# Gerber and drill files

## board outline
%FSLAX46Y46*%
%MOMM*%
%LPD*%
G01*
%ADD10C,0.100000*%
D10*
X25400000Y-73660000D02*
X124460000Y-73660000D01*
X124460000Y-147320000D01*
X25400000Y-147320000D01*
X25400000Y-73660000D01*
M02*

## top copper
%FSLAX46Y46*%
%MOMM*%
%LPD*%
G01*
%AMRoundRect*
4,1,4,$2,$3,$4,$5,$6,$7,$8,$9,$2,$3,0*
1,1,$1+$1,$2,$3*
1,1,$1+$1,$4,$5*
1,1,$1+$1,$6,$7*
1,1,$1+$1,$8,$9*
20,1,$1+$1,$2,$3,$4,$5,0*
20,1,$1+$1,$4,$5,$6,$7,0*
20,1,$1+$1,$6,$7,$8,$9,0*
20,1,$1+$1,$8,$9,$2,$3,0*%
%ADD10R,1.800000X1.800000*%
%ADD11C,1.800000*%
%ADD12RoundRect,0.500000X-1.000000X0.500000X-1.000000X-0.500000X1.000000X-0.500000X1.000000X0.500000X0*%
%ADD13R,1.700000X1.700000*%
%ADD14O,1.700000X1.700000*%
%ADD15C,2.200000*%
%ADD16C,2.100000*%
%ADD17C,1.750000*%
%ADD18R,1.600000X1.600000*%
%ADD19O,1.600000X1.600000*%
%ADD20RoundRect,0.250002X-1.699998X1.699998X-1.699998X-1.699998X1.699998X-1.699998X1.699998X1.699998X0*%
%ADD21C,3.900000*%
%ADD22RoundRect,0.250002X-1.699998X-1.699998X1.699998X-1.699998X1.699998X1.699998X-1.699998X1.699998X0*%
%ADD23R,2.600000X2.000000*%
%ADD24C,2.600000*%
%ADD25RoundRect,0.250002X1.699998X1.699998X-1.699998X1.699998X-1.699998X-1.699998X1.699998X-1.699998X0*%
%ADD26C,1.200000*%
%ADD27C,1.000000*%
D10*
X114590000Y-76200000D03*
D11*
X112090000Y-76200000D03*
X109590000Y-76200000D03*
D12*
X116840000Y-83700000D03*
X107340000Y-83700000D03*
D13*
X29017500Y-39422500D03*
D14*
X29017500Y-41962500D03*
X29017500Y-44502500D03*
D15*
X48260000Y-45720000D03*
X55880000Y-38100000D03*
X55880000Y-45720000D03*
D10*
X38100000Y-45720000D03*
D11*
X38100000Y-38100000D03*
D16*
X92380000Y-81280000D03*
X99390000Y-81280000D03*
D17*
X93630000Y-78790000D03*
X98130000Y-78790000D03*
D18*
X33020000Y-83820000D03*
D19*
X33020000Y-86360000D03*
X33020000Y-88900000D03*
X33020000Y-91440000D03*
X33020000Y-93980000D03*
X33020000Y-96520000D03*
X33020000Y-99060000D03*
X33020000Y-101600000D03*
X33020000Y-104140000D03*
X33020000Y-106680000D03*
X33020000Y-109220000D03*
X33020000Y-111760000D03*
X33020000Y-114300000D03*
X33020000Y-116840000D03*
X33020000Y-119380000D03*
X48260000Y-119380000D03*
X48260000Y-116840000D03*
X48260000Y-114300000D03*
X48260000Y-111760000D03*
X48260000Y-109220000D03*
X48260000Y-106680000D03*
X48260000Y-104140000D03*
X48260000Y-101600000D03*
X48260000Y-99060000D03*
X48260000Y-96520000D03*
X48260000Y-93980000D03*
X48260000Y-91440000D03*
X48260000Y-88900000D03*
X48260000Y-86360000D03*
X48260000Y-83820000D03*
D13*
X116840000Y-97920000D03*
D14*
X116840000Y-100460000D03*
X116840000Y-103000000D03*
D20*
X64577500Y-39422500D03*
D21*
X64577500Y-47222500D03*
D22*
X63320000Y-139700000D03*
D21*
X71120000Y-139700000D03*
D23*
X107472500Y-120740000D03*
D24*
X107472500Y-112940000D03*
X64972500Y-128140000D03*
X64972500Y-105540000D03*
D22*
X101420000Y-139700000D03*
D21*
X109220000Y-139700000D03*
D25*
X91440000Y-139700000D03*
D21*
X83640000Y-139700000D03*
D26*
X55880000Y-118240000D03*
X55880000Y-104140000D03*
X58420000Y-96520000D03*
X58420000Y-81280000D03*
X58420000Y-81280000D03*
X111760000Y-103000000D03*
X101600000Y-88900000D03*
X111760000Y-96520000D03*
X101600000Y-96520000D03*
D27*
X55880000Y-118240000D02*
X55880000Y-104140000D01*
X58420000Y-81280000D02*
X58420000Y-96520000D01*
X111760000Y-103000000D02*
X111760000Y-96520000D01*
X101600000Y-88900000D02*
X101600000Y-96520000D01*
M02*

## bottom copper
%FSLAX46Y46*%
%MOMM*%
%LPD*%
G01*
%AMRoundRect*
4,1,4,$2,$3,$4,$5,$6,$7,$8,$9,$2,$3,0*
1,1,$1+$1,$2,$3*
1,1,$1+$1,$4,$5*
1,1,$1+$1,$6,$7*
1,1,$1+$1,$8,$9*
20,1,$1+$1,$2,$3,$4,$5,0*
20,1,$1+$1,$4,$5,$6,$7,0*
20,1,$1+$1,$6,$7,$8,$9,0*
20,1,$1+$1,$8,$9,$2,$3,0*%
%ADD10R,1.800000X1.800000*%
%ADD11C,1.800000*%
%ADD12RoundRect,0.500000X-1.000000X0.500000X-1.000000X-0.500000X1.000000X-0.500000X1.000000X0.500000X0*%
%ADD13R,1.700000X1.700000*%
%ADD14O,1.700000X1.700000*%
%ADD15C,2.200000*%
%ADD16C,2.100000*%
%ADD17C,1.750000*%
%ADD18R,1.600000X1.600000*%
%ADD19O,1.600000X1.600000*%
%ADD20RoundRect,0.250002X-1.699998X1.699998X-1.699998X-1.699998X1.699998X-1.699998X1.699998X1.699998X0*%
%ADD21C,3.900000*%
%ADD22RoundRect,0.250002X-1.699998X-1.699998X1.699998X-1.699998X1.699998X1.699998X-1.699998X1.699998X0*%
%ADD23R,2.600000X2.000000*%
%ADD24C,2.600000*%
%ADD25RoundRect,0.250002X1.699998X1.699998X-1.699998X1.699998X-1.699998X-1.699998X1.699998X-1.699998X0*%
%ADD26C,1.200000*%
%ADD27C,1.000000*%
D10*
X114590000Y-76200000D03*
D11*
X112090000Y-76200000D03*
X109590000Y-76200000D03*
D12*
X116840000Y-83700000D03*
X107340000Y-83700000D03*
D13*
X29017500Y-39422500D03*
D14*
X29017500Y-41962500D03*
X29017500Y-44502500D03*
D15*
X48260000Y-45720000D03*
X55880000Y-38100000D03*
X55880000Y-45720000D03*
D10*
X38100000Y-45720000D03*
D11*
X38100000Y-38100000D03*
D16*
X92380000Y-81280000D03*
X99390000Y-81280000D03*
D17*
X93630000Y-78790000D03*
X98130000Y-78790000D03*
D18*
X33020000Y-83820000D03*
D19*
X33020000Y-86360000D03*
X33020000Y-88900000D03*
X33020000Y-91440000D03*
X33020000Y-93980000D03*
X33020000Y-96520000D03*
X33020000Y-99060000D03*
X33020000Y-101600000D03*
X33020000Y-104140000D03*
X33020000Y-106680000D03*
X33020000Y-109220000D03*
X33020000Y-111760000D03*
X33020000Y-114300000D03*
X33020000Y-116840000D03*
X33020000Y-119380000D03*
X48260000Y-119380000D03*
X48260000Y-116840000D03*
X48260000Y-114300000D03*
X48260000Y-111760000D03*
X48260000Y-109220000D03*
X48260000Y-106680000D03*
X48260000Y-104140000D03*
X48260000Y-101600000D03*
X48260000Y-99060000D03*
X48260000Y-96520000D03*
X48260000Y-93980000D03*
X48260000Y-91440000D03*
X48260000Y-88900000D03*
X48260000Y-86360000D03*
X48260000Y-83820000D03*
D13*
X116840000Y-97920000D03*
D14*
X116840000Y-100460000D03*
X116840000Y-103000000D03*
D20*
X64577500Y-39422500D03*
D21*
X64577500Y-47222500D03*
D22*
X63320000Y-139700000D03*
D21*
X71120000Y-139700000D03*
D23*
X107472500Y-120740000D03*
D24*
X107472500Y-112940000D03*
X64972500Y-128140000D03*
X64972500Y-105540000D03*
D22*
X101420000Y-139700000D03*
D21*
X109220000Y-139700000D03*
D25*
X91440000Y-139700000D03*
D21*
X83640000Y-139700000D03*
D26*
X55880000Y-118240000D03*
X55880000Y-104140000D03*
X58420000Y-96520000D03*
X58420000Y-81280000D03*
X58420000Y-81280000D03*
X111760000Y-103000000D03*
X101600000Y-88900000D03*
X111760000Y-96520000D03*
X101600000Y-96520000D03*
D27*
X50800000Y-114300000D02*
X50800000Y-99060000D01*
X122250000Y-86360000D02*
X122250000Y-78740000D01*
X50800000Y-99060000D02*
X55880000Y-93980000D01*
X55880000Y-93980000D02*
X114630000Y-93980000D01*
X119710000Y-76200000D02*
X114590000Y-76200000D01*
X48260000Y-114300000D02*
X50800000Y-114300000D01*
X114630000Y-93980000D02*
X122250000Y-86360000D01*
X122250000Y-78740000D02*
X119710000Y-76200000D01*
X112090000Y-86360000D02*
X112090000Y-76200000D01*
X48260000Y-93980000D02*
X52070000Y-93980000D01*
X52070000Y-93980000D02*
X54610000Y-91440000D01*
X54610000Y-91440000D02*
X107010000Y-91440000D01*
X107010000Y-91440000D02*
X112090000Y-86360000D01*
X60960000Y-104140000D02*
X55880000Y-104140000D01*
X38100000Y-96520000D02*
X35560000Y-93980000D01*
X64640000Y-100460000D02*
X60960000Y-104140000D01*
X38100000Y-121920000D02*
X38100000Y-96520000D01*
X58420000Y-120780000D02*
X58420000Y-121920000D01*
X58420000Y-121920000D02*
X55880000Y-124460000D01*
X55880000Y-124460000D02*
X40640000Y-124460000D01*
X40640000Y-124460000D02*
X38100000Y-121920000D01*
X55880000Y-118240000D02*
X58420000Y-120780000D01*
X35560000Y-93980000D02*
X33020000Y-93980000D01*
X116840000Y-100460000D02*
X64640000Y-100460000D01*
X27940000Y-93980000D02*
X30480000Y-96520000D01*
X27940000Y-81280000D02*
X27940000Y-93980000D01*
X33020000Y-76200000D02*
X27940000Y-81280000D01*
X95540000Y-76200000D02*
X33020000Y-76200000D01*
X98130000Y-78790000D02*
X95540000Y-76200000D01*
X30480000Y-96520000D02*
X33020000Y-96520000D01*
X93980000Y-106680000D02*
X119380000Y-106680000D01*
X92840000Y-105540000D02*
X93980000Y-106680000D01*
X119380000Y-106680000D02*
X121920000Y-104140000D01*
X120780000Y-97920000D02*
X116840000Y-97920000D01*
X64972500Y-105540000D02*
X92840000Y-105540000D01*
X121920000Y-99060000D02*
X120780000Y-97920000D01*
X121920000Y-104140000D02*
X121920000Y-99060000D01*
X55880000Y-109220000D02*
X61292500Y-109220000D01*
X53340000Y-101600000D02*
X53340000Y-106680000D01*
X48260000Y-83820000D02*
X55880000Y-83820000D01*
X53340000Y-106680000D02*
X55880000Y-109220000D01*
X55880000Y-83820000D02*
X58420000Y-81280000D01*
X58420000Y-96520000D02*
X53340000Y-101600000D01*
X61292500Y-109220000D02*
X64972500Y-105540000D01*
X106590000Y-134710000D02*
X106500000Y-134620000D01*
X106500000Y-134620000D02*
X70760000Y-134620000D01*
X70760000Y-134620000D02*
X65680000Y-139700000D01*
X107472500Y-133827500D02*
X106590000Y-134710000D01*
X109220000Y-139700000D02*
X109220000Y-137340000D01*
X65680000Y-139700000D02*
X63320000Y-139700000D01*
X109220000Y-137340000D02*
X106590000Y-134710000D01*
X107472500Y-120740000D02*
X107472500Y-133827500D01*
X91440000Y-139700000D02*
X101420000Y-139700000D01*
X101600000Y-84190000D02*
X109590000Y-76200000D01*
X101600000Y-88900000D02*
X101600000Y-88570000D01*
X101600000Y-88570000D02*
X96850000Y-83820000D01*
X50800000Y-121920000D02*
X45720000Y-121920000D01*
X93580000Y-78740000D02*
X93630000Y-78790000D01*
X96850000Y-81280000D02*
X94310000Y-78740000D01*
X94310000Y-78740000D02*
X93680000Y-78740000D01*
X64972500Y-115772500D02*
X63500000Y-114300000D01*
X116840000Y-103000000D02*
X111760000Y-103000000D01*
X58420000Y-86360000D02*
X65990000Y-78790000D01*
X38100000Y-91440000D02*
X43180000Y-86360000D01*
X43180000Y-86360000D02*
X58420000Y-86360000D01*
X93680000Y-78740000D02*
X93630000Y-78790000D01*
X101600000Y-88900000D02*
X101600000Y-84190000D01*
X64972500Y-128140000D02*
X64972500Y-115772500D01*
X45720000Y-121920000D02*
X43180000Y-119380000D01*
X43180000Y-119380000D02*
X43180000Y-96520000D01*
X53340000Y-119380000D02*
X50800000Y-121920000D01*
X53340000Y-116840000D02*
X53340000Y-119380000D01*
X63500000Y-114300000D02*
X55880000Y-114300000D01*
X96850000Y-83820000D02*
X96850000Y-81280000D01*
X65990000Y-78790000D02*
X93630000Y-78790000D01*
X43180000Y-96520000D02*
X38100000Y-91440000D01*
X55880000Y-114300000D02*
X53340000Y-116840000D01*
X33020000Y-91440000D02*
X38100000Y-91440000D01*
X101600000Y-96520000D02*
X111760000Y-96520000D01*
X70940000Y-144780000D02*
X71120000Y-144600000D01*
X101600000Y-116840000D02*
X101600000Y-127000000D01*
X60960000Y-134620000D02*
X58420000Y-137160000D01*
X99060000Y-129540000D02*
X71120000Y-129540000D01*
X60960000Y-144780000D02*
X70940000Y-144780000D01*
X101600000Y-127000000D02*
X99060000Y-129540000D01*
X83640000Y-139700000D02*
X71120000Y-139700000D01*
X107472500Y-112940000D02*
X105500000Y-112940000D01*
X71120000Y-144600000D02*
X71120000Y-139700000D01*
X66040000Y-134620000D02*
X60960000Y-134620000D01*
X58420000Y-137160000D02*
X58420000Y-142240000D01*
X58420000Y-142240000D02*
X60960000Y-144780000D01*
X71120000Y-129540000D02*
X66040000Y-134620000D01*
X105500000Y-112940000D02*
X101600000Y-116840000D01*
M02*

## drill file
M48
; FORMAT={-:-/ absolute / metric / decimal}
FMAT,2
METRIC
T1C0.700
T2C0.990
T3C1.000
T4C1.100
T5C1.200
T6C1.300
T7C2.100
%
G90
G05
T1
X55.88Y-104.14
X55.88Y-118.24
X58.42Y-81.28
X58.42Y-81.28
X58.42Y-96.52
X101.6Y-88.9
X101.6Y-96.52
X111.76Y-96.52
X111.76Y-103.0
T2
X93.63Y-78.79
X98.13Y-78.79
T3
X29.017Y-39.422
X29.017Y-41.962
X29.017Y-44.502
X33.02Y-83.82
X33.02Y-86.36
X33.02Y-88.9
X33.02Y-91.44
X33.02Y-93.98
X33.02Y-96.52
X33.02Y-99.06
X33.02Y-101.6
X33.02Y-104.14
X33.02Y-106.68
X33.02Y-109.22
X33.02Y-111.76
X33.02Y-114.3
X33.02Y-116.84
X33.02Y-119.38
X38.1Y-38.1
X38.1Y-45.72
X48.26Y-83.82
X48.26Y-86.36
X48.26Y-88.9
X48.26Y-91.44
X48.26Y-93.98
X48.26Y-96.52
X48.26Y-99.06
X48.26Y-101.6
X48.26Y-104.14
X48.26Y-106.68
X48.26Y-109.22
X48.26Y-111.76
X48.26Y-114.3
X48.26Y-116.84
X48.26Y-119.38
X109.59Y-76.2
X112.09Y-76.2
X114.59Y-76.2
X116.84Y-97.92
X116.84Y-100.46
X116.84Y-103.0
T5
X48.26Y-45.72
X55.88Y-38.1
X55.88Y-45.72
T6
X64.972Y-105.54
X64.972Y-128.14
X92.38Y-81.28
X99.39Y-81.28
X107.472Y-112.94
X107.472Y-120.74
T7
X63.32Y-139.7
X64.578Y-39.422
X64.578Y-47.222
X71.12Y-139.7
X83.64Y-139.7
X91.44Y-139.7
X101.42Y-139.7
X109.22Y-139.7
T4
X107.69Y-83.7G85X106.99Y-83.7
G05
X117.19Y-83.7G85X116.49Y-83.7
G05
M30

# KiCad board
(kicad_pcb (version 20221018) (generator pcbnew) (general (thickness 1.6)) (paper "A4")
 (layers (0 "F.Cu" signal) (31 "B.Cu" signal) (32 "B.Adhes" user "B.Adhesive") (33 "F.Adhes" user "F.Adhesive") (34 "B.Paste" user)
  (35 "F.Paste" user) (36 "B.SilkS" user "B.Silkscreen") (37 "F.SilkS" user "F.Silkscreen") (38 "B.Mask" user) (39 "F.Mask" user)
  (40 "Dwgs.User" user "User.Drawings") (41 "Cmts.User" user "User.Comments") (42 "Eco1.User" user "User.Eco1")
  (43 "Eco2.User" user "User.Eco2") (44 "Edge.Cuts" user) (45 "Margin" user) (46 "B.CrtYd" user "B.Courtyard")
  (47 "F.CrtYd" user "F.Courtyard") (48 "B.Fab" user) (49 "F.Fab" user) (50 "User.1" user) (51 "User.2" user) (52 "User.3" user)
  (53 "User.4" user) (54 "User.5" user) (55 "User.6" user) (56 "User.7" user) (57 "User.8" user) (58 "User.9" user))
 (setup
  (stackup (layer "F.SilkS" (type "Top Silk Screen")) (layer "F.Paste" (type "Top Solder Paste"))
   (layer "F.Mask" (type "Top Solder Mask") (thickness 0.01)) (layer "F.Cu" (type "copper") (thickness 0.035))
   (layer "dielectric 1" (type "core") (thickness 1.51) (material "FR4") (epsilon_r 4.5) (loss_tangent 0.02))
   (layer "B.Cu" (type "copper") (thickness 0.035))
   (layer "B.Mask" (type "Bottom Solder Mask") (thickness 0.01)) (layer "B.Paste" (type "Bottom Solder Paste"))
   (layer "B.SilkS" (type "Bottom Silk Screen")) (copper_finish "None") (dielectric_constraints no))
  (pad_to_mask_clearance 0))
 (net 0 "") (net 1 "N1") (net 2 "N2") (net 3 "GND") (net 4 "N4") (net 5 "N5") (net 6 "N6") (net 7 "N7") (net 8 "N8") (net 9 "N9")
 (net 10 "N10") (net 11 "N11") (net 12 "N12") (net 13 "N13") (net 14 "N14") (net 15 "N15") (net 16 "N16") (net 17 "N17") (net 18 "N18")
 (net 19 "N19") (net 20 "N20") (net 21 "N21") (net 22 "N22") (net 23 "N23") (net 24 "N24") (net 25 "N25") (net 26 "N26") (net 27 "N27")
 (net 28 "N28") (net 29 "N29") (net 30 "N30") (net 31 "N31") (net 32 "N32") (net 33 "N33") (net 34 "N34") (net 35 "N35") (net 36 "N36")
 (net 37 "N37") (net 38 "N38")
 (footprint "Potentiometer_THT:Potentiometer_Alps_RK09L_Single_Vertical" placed (layer "F.Cu") (at 114.59 76.2 -90)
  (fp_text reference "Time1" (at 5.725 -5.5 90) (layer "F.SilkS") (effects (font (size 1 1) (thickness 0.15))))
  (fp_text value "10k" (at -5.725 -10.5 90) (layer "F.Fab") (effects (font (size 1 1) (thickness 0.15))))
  (pad "1" thru_hole rect (at 0 0 270) (size 1.8 1.8) (drill 1) (layers "*.Cu" "*.Mask") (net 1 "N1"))
  (pad "2" thru_hole circle (at 0 2.5 270) (size 1.8 1.8) (drill 1) (layers "*.Cu" "*.Mask") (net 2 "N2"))
  (pad "3" thru_hole circle (at 0 5 270) (size 1.8 1.8) (drill 1) (layers "*.Cu" "*.Mask") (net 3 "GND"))
  (pad "MP" thru_hole roundrect (at 7.5 -2.25 270) (size 2 3) (drill oval 1.1 1.8) (layers "*.Cu" "*.Mask") (roundrect_rratio 0.25))
  (pad "MP" thru_hole roundrect (at 7.5 7.25 270) (size 2 3) (drill oval 1.1 1.8) (layers "*.Cu" "*.Mask") (roundrect_rratio 0.25))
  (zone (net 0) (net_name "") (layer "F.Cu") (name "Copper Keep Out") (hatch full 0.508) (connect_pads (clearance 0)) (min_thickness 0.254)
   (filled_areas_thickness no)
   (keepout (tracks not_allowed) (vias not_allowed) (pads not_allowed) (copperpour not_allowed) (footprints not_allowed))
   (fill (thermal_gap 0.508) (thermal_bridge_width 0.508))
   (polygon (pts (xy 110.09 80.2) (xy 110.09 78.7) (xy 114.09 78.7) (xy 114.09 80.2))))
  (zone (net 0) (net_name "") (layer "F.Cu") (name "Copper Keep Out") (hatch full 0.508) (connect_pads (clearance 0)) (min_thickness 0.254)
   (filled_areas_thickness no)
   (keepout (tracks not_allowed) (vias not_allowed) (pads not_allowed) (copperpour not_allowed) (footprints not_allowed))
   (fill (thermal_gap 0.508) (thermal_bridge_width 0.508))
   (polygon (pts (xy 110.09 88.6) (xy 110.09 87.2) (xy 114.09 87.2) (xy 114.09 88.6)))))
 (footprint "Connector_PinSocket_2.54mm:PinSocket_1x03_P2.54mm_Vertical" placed (layer "F.Cu") (at 29.0175 39.4225)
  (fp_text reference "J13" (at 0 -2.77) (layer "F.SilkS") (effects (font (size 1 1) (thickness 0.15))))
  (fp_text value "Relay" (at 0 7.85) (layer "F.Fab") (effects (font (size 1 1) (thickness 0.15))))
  (pad "1" thru_hole rect (at 0 0) (size 1.7 1.7) (drill 1) (layers "*.Cu" "*.Mask") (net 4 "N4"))
  (pad "2" thru_hole oval (at 0 2.54) (size 1.7 1.7) (drill 1) (layers "*.Cu" "*.Mask") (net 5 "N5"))
  (pad "3" thru_hole oval (at 0 5.08) (size 1.7 1.7) (drill 1) (layers "*.Cu" "*.Mask") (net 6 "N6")))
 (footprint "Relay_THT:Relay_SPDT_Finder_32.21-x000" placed (layer "F.Cu") (at 38.1 45.72)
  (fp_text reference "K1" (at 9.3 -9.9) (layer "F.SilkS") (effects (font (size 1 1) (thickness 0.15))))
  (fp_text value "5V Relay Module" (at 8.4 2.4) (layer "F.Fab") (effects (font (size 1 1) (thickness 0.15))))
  (pad "11" thru_hole circle (at 10.16 0 90) (size 2.2 2.2) (drill 1.2) (layers "*.Cu" "*.Mask") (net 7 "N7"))
  (pad "12" thru_hole circle (at 17.78 -7.62 90) (size 2.2 2.2) (drill 1.2) (layers "*.Cu" "*.Mask") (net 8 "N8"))
  (pad "14" thru_hole circle (at 17.78 0 90) (size 2.2 2.2) (drill 1.2) (layers "*.Cu" "*.Mask") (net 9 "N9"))
  (pad "A1" thru_hole rect (at 0 0 90) (size 1.8 1.8) (drill 1) (layers "*.Cu" "*.Mask") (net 6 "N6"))
  (pad "A2" thru_hole circle (at 0 -7.62 90) (size 1.8 1.8) (drill 1) (layers "*.Cu" "*.Mask") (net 5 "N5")))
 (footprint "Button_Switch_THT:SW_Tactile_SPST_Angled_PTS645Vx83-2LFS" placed (layer "F.Cu") (at 93.63 78.79)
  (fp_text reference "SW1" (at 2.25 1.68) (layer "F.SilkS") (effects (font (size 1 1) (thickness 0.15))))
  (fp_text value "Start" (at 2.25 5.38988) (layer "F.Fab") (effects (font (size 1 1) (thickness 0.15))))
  (pad "" thru_hole circle (at -1.25 2.49) (size 2.1 2.1) (drill 1.3) (layers "*.Cu" "*.Mask"))
  (pad "" thru_hole circle (at 5.76 2.49) (size 2.1 2.1) (drill 1.3) (layers "*.Cu" "*.Mask"))
  (pad "1" thru_hole circle (at 0 0) (size 1.75 1.75) (drill 0.99) (layers "*.Cu" "*.Mask") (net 3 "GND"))
  (pad "2" thru_hole circle (at 4.5 0) (size 1.75 1.75) (drill 0.99) (layers "*.Cu" "*.Mask") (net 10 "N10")))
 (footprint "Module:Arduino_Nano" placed (layer "F.Cu") (at 33.02 83.82)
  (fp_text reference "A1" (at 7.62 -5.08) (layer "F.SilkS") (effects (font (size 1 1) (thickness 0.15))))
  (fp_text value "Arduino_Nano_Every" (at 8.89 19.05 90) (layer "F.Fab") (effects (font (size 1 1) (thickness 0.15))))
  (pad "1" thru_hole rect (at 0 0) (size 1.6 1.6) (drill 1) (layers "*.Cu" "*.Mask") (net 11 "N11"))
  (pad "2" thru_hole oval (at 0 2.54) (size 1.6 1.6) (drill 1) (layers "*.Cu" "*.Mask") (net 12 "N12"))
  (pad "3" thru_hole oval (at 0 5.08) (size 1.6 1.6) (drill 1) (layers "*.Cu" "*.Mask") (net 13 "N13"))
  (pad "4" thru_hole oval (at 0 7.62) (size 1.6 1.6) (drill 1) (layers "*.Cu" "*.Mask") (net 3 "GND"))
  (pad "5" thru_hole oval (at 0 10.16) (size 1.6 1.6) (drill 1) (layers "*.Cu" "*.Mask") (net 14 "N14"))
  (pad "6" thru_hole oval (at 0 12.7) (size 1.6 1.6) (drill 1) (layers "*.Cu" "*.Mask") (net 10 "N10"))
  (pad "7" thru_hole oval (at 0 15.24) (size 1.6 1.6) (drill 1) (layers "*.Cu" "*.Mask") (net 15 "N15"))
  (pad "8" thru_hole oval (at 0 17.78) (size 1.6 1.6) (drill 1) (layers "*.Cu" "*.Mask") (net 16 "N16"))
  (pad "9" thru_hole oval (at 0 20.32) (size 1.6 1.6) (drill 1) (layers "*.Cu" "*.Mask") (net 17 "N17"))
  (pad "10" thru_hole oval (at 0 22.86) (size 1.6 1.6) (drill 1) (layers "*.Cu" "*.Mask") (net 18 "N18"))
  (pad "11" thru_hole oval (at 0 25.4) (size 1.6 1.6) (drill 1) (layers "*.Cu" "*.Mask") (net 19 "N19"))
  (pad "12" thru_hole oval (at 0 27.94) (size 1.6 1.6) (drill 1) (layers "*.Cu" "*.Mask") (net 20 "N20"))
  (pad "13" thru_hole oval (at 0 30.48) (size 1.6 1.6) (drill 1) (layers "*.Cu" "*.Mask") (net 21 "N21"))
  (pad "14" thru_hole oval (at 0 33.02) (size 1.6 1.6) (drill 1) (layers "*.Cu" "*.Mask") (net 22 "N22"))
  (pad "15" thru_hole oval (at 0 35.56) (size 1.6 1.6) (drill 1) (layers "*.Cu" "*.Mask") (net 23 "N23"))
  (pad "16" thru_hole oval (at 15.24 35.56) (size 1.6 1.6) (drill 1) (layers "*.Cu" "*.Mask") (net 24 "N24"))
  (pad "17" thru_hole oval (at 15.24 33.02) (size 1.6 1.6) (drill 1) (layers "*.Cu" "*.Mask") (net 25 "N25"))
  (pad "18" thru_hole oval (at 15.24 30.48) (size 1.6 1.6) (drill 1) (layers "*.Cu" "*.Mask") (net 1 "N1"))
  (pad "19" thru_hole oval (at 15.24 27.94) (size 1.6 1.6) (drill 1) (layers "*.Cu" "*.Mask") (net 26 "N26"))
  (pad "20" thru_hole oval (at 15.24 25.4) (size 1.6 1.6) (drill 1) (layers "*.Cu" "*.Mask") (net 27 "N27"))
  (pad "21" thru_hole oval (at 15.24 22.86) (size 1.6 1.6) (drill 1) (layers "*.Cu" "*.Mask") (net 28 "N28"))
  (pad "22" thru_hole oval (at 15.24 20.32) (size 1.6 1.6) (drill 1) (layers "*.Cu" "*.Mask") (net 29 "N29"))
  (pad "23" thru_hole oval (at 15.24 17.78) (size 1.6 1.6) (drill 1) (layers "*.Cu" "*.Mask") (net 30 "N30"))
  (pad "24" thru_hole oval (at 15.24 15.24) (size 1.6 1.6) (drill 1) (layers "*.Cu" "*.Mask") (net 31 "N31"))
  (pad "25" thru_hole oval (at 15.24 12.7) (size 1.6 1.6) (drill 1) (layers "*.Cu" "*.Mask") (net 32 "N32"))
  (pad "26" thru_hole oval (at 15.24 10.16) (size 1.6 1.6) (drill 1) (layers "*.Cu" "*.Mask") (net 2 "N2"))
  (pad "27" thru_hole oval (at 15.24 7.62) (size 1.6 1.6) (drill 1) (layers "*.Cu" "*.Mask") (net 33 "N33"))
  (pad "28" thru_hole oval (at 15.24 5.08) (size 1.6 1.6) (drill 1) (layers "*.Cu" "*.Mask") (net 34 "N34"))
  (pad "29" thru_hole oval (at 15.24 2.54) (size 1.6 1.6) (drill 1) (layers "*.Cu" "*.Mask") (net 3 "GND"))
  (pad "30" thru_hole oval (at 15.24 0) (size 1.6 1.6) (drill 1) (layers "*.Cu" "*.Mask") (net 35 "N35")))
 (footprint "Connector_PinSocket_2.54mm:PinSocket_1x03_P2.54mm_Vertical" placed (layer "F.Cu") (at 116.84 97.92)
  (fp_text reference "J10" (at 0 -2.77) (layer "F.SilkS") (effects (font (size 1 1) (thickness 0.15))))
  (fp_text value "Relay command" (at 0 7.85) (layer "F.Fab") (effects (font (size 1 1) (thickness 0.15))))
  (pad "1" thru_hole rect (at 0 0) (size 1.7 1.7) (drill 1) (layers "*.Cu" "*.Mask") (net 35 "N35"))
  (pad "2" thru_hole oval (at 0 2.54) (size 1.7 1.7) (drill 1) (layers "*.Cu" "*.Mask") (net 14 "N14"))
  (pad "3" thru_hole oval (at 0 5.08) (size 1.7 1.7) (drill 1) (layers "*.Cu" "*.Mask") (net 3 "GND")))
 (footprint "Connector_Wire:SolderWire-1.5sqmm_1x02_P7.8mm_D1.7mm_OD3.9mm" (layer "F.Cu") (at 64.5775 39.4225 -90)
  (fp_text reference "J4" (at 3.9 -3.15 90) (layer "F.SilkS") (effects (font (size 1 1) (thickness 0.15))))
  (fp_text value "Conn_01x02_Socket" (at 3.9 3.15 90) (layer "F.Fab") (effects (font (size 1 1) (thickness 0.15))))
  (pad "1" thru_hole roundrect (at 0 0 270) (size 3.9 3.9) (drill 2.1) (layers "*.Cu" "*.Mask") (roundrect_rratio 0.064103) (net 7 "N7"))
  (pad "2" thru_hole circle (at 7.8 0 270) (size 3.9 3.9) (drill 2.1) (layers "*.Cu" "*.Mask") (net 9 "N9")))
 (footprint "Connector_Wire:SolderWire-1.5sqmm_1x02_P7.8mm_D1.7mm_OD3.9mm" (layer "F.Cu") (at 63.32 139.7)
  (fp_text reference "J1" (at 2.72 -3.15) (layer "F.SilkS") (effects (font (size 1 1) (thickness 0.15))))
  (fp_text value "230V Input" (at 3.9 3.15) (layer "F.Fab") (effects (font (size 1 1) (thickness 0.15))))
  (pad "1" thru_hole roundrect (at 0 0) (size 3.9 3.9) (drill 2.1) (layers "*.Cu" "*.Mask") (roundrect_rratio 0.064103) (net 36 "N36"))
  (pad "2" thru_hole circle (at 7.8 0) (size 3.9 3.9) (drill 2.1) (layers "*.Cu" "*.Mask") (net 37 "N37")))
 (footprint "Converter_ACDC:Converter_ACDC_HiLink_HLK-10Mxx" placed (layer "F.Cu") (at 107.4725 120.74 180)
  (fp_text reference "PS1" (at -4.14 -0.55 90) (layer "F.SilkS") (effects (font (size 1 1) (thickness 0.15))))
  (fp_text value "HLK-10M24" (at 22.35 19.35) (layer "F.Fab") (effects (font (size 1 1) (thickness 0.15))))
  (pad "1" thru_hole rect (at 0 0 180) (size 2.6 2) (drill 1.3) (layers "*.Cu" "*.Mask") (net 36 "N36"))
  (pad "2" thru_hole circle (at 0 7.8 180) (size 2.6 2.6) (drill 1.3) (layers "*.Cu" "*.Mask") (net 37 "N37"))
  (pad "3" thru_hole circle (at 42.5 -7.4 180) (size 2.6 2.6) (drill 1.3) (layers "*.Cu" "*.Mask") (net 3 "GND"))
  (pad "4" thru_hole circle (at 42.5 15.2 180) (size 2.6 2.6) (drill 1.3) (layers "*.Cu" "*.Mask") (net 35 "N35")))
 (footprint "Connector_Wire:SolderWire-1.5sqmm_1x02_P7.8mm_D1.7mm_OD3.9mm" (layer "F.Cu") (at 101.42 139.7)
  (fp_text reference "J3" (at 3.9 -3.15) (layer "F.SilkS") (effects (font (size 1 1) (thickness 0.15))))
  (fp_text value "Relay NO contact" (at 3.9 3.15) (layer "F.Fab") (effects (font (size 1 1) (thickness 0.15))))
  (pad "1" thru_hole roundrect (at 0 0) (size 3.9 3.9) (drill 2.1) (layers "*.Cu" "*.Mask") (roundrect_rratio 0.064103) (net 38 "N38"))
  (pad "2" thru_hole circle (at 7.8 0) (size 3.9 3.9) (drill 2.1) (layers "*.Cu" "*.Mask") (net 36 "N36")))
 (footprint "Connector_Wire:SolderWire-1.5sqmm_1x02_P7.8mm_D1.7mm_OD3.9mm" (layer "F.Cu") (at 91.44 139.7 180)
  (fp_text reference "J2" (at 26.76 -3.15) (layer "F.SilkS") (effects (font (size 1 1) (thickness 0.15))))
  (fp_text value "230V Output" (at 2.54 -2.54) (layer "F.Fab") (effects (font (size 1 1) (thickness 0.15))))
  (pad "1" thru_hole roundrect (at 0 0 180) (size 3.9 3.9) (drill 2.1) (layers "*.Cu" "*.Mask") (roundrect_rratio 0.064103) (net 38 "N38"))
  (pad "2" thru_hole circle (at 7.8 0 180) (size 3.9 3.9) (drill 2.1) (layers "*.Cu" "*.Mask") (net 37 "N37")))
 (gr_rect (start 25.4 73.66) (end 124.46 147.32) (stroke (width 0.1) (type default)) (fill none) (layer "Edge.Cuts"))
 (segment (start 50.8 114.3) (end 50.8 99.06) (width 1) (layer "B.Cu") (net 1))
 (segment (start 122.25 86.36) (end 122.25 78.74) (width 1) (layer "B.Cu") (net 1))
 (segment (start 50.8 99.06) (end 55.88 93.98) (width 1) (layer "B.Cu") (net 1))
 (segment (start 55.88 93.98) (end 114.63 93.98) (width 1) (layer "B.Cu") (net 1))
 (segment (start 119.71 76.2) (end 114.59 76.2) (width 1) (layer "B.Cu") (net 1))
 (segment (start 48.26 114.3) (end 50.8 114.3) (width 1) (layer "B.Cu") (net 1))
 (segment (start 114.63 93.98) (end 122.25 86.36) (width 1) (layer "B.Cu") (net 1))
 (segment (start 122.25 78.74) (end 119.71 76.2) (width 1) (layer "B.Cu") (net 1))
 (segment (start 112.09 86.36) (end 112.09 76.2) (width 1) (layer "B.Cu") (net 2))
 (segment (start 48.26 93.98) (end 52.07 93.98) (width 1) (layer "B.Cu") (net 2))
 (segment (start 52.07 93.98) (end 54.61 91.44) (width 1) (layer "B.Cu") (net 2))
 (segment (start 54.61 91.44) (end 107.01 91.44) (width 1) (layer "B.Cu") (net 2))
 (segment (start 107.01 91.44) (end 112.09 86.36) (width 1) (layer "B.Cu") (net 2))
 (segment (start 55.88 118.24) (end 55.88 104.14) (width 1) (layer "F.Cu") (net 14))
 (via (at 55.88 118.24) (size 1.2) (drill 0.7) (layers "F.Cu" "B.Cu") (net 14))
 (via (at 55.88 104.14) (size 1.2) (drill 0.7) (layers "F.Cu" "B.Cu") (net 14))
 (segment (start 60.96 104.14) (end 55.88 104.14) (width 1) (layer "B.Cu") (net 14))
 (segment (start 38.1 96.52) (end 35.56 93.98) (width 1) (layer "B.Cu") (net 14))
 (segment (start 64.64 100.46) (end 60.96 104.14) (width 1) (layer "B.Cu") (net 14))
 (segment (start 38.1 121.92) (end 38.1 96.52) (width 1) (layer "B.Cu") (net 14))
 (segment (start 58.42 120.78) (end 58.42 121.92) (width 1) (layer "B.Cu") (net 14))
 (segment (start 58.42 121.92) (end 55.88 124.46) (width 1) (layer "B.Cu") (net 14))
 (segment (start 55.88 124.46) (end 40.64 124.46) (width 1) (layer "B.Cu") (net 14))
 (segment (start 40.64 124.46) (end 38.1 121.92) (width 1) (layer "B.Cu") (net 14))
 (segment (start 55.88 118.24) (end 58.42 120.78) (width 1) (layer "B.Cu") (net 14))
 (segment (start 35.56 93.98) (end 33.02 93.98) (width 1) (layer "B.Cu") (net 14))
 (segment (start 116.84 100.46) (end 64.64 100.46) (width 1) (layer "B.Cu") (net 14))
 (segment (start 27.94 93.98) (end 30.48 96.52) (width 1) (layer "B.Cu") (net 10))
 (segment (start 27.94 81.28) (end 27.94 93.98) (width 1) (layer "B.Cu") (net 10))
 (segment (start 33.02 76.2) (end 27.94 81.28) (width 1) (layer "B.Cu") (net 10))
 (segment (start 95.54 76.2) (end 33.02 76.2) (width 1) (layer "B.Cu") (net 10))
 (segment (start 98.13 78.79) (end 95.54 76.2) (width 1) (layer "B.Cu") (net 10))
 (segment (start 30.48 96.52) (end 33.02 96.52) (width 1) (layer "B.Cu") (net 10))
 (segment (start 58.42 81.28) (end 58.42 96.52) (width 1) (layer "F.Cu") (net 35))
 (via (at 58.42 96.52) (size 1.2) (drill 0.7) (layers "F.Cu" "B.Cu") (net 35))
 (via (at 58.42 81.28) (size 1.2) (drill 0.7) (layers "F.Cu" "B.Cu") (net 35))
 (via (at 58.42 81.28) (size 1.2) (drill 0.7) (layers "F.Cu" "B.Cu") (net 35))
 (segment (start 93.98 106.68) (end 119.38 106.68) (width 1) (layer "B.Cu") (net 35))
 (segment (start 92.84 105.54) (end 93.98 106.68) (width 1) (layer "B.Cu") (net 35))
 (segment (start 119.38 106.68) (end 121.92 104.14) (width 1) (layer "B.Cu") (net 35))
 (segment (start 120.78 97.92) (end 116.84 97.92) (width 1) (layer "B.Cu") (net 35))
 (segment (start 64.9725 105.54) (end 92.84 105.54) (width 1) (layer "B.Cu") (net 35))
 (segment (start 121.92 99.06) (end 120.78 97.92) (width 1) (layer "B.Cu") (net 35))
 (segment (start 121.92 104.14) (end 121.92 99.06) (width 1) (layer "B.Cu") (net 35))
 (segment (start 55.88 109.22) (end 61.2925 109.22) (width 1) (layer "B.Cu") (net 35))
 (segment (start 53.34 101.6) (end 53.34 106.68) (width 1) (layer "B.Cu") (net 35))
 (segment (start 48.26 83.82) (end 55.88 83.82) (width 1) (layer "B.Cu") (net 35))
 (segment (start 53.34 106.68) (end 55.88 109.22) (width 1) (layer "B.Cu") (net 35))
 (segment (start 55.88 83.82) (end 58.42 81.28) (width 1) (layer "B.Cu") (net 35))
 (segment (start 58.42 96.52) (end 53.34 101.6) (width 1) (layer "B.Cu") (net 35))
 (segment (start 61.2925 109.22) (end 64.9725 105.54) (width 1) (layer "B.Cu") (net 35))
 (segment (start 106.59 134.71) (end 106.5 134.62) (width 1) (layer "B.Cu") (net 36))
 (segment (start 106.5 134.62) (end 70.76 134.62) (width 1) (layer "B.Cu") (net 36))
 (segment (start 70.76 134.62) (end 65.68 139.7) (width 1) (layer "B.Cu") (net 36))
 (segment (start 107.4725 133.8275) (end 106.59 134.71) (width 1) (layer "B.Cu") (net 36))
 (segment (start 109.22 139.7) (end 109.22 137.34) (width 1) (layer "B.Cu") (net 36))
 (segment (start 65.68 139.7) (end 63.32 139.7) (width 1) (layer "B.Cu") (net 36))
 (segment (start 109.22 137.34) (end 106.59 134.71) (width 1) (layer "B.Cu") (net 36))
 (segment (start 107.4725 120.74) (end 107.4725 133.8275) (width 1) (layer "B.Cu") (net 36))
 (segment (start 91.44 139.7) (end 101.42 139.7) (width 1) (layer "B.Cu") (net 38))
 (segment (start 111.76 103) (end 111.76 96.52) (width 1) (layer "F.Cu") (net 3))
 (segment (start 101.6 88.9) (end 101.6 96.52) (width 1) (layer "F.Cu") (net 3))
 (via (at 111.76 103) (size 1.2) (drill 0.7) (layers "F.Cu" "B.Cu") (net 3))
 (via (at 101.6 88.9) (size 1.2) (drill 0.7) (layers "F.Cu" "B.Cu") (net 3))
 (via (at 111.76 96.52) (size 1.2) (drill 0.7) (layers "F.Cu" "B.Cu") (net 3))
 (via (at 101.6 96.52) (size 1.2) (drill 0.7) (layers "F.Cu" "B.Cu") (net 3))
 (segment (start 101.6 84.19) (end 109.59 76.2) (width 1) (layer "B.Cu") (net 3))
 (segment (start 101.6 88.9) (end 101.6 88.57) (width 1) (layer "B.Cu") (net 3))
 (segment (start 101.6 88.57) (end 96.85 83.82) (width 1) (layer "B.Cu") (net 3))
 (segment (start 50.8 121.92) (end 45.72 121.92) (width 1) (layer "B.Cu") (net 3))
 (segment (start 93.58 78.74) (end 93.63 78.79) (width 1) (layer "B.Cu") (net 3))
 (segment (start 96.85 81.28) (end 94.31 78.74) (width 1) (layer "B.Cu") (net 3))
 (segment (start 94.31 78.74) (end 93.68 78.74) (width 1) (layer "B.Cu") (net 3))
 (segment (start 64.9725 115.7725) (end 63.5 114.3) (width 1) (layer "B.Cu") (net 3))
 (segment (start 116.84 103) (end 111.76 103) (width 1) (layer "B.Cu") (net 3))
 (segment (start 58.42 86.36) (end 65.99 78.79) (width 1) (layer "B.Cu") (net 3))
 (segment (start 38.1 91.44) (end 43.18 86.36) (width 1) (layer "B.Cu") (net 3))
 (segment (start 43.18 86.36) (end 58.42 86.36) (width 1) (layer "B.Cu") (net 3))
 (segment (start 93.68 78.74) (end 93.63 78.79) (width 1) (layer "B.Cu") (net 3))
 (segment (start 101.6 88.9) (end 101.6 84.19) (width 1) (layer "B.Cu") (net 3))
 (segment (start 64.9725 128.14) (end 64.9725 115.7725) (width 1) (layer "B.Cu") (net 3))
 (segment (start 45.72 121.92) (end 43.18 119.38) (width 1) (layer "B.Cu") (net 3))
 (segment (start 43.18 119.38) (end 43.18 96.52) (width 1) (layer "B.Cu") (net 3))
 (segment (start 53.34 119.38) (end 50.8 121.92) (width 1) (layer "B.Cu") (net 3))
 (segment (start 53.34 116.84) (end 53.34 119.38) (width 1) (layer "B.Cu") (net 3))
 (segment (start 63.5 114.3) (end 55.88 114.3) (width 1) (layer "B.Cu") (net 3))
 (segment (start 96.85 83.82) (end 96.85 81.28) (width 1) (layer "B.Cu") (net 3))
 (segment (start 65.99 78.79) (end 93.63 78.79) (width 1) (layer "B.Cu") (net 3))
 (segment (start 43.18 96.52) (end 38.1 91.44) (width 1) (layer "B.Cu") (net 3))
 (segment (start 55.88 114.3) (end 53.34 116.84) (width 1) (layer "B.Cu") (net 3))
 (segment (start 33.02 91.44) (end 38.1 91.44) (width 1) (layer "B.Cu") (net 3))
 (segment (start 101.6 96.52) (end 111.76 96.52) (width 1) (layer "B.Cu") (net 3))
 (segment (start 70.94 144.78) (end 71.12 144.6) (width 1) (layer "B.Cu") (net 37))
 (segment (start 101.6 116.84) (end 101.6 127) (width 1) (layer "B.Cu") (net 37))
 (segment (start 60.96 134.62) (end 58.42 137.16) (width 1) (layer "B.Cu") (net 37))
 (segment (start 99.06 129.54) (end 71.12 129.54) (width 1) (layer "B.Cu") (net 37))
 (segment (start 60.96 144.78) (end 70.94 144.78) (width 1) (layer "B.Cu") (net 37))
 (segment (start 101.6 127) (end 99.06 129.54) (width 1) (layer "B.Cu") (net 37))
 (segment (start 83.64 139.7) (end 71.12 139.7) (width 1) (layer "B.Cu") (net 37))
 (segment (start 107.4725 112.94) (end 105.5 112.94) (width 1) (layer "B.Cu") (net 37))
 (segment (start 71.12 144.6) (end 71.12 139.7) (width 1) (layer "B.Cu") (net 37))
 (segment (start 66.04 134.62) (end 60.96 134.62) (width 1) (layer "B.Cu") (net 37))
 (segment (start 58.42 137.16) (end 58.42 142.24) (width 1) (layer "B.Cu") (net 37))
 (segment (start 58.42 142.24) (end 60.96 144.78) (width 1) (layer "B.Cu") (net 37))
 (segment (start 71.12 129.54) (end 66.04 134.62) (width 1) (layer "B.Cu") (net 37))
 (segment (start 105.5 112.94) (end 101.6 116.84) (width 1) (layer "B.Cu") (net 37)))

